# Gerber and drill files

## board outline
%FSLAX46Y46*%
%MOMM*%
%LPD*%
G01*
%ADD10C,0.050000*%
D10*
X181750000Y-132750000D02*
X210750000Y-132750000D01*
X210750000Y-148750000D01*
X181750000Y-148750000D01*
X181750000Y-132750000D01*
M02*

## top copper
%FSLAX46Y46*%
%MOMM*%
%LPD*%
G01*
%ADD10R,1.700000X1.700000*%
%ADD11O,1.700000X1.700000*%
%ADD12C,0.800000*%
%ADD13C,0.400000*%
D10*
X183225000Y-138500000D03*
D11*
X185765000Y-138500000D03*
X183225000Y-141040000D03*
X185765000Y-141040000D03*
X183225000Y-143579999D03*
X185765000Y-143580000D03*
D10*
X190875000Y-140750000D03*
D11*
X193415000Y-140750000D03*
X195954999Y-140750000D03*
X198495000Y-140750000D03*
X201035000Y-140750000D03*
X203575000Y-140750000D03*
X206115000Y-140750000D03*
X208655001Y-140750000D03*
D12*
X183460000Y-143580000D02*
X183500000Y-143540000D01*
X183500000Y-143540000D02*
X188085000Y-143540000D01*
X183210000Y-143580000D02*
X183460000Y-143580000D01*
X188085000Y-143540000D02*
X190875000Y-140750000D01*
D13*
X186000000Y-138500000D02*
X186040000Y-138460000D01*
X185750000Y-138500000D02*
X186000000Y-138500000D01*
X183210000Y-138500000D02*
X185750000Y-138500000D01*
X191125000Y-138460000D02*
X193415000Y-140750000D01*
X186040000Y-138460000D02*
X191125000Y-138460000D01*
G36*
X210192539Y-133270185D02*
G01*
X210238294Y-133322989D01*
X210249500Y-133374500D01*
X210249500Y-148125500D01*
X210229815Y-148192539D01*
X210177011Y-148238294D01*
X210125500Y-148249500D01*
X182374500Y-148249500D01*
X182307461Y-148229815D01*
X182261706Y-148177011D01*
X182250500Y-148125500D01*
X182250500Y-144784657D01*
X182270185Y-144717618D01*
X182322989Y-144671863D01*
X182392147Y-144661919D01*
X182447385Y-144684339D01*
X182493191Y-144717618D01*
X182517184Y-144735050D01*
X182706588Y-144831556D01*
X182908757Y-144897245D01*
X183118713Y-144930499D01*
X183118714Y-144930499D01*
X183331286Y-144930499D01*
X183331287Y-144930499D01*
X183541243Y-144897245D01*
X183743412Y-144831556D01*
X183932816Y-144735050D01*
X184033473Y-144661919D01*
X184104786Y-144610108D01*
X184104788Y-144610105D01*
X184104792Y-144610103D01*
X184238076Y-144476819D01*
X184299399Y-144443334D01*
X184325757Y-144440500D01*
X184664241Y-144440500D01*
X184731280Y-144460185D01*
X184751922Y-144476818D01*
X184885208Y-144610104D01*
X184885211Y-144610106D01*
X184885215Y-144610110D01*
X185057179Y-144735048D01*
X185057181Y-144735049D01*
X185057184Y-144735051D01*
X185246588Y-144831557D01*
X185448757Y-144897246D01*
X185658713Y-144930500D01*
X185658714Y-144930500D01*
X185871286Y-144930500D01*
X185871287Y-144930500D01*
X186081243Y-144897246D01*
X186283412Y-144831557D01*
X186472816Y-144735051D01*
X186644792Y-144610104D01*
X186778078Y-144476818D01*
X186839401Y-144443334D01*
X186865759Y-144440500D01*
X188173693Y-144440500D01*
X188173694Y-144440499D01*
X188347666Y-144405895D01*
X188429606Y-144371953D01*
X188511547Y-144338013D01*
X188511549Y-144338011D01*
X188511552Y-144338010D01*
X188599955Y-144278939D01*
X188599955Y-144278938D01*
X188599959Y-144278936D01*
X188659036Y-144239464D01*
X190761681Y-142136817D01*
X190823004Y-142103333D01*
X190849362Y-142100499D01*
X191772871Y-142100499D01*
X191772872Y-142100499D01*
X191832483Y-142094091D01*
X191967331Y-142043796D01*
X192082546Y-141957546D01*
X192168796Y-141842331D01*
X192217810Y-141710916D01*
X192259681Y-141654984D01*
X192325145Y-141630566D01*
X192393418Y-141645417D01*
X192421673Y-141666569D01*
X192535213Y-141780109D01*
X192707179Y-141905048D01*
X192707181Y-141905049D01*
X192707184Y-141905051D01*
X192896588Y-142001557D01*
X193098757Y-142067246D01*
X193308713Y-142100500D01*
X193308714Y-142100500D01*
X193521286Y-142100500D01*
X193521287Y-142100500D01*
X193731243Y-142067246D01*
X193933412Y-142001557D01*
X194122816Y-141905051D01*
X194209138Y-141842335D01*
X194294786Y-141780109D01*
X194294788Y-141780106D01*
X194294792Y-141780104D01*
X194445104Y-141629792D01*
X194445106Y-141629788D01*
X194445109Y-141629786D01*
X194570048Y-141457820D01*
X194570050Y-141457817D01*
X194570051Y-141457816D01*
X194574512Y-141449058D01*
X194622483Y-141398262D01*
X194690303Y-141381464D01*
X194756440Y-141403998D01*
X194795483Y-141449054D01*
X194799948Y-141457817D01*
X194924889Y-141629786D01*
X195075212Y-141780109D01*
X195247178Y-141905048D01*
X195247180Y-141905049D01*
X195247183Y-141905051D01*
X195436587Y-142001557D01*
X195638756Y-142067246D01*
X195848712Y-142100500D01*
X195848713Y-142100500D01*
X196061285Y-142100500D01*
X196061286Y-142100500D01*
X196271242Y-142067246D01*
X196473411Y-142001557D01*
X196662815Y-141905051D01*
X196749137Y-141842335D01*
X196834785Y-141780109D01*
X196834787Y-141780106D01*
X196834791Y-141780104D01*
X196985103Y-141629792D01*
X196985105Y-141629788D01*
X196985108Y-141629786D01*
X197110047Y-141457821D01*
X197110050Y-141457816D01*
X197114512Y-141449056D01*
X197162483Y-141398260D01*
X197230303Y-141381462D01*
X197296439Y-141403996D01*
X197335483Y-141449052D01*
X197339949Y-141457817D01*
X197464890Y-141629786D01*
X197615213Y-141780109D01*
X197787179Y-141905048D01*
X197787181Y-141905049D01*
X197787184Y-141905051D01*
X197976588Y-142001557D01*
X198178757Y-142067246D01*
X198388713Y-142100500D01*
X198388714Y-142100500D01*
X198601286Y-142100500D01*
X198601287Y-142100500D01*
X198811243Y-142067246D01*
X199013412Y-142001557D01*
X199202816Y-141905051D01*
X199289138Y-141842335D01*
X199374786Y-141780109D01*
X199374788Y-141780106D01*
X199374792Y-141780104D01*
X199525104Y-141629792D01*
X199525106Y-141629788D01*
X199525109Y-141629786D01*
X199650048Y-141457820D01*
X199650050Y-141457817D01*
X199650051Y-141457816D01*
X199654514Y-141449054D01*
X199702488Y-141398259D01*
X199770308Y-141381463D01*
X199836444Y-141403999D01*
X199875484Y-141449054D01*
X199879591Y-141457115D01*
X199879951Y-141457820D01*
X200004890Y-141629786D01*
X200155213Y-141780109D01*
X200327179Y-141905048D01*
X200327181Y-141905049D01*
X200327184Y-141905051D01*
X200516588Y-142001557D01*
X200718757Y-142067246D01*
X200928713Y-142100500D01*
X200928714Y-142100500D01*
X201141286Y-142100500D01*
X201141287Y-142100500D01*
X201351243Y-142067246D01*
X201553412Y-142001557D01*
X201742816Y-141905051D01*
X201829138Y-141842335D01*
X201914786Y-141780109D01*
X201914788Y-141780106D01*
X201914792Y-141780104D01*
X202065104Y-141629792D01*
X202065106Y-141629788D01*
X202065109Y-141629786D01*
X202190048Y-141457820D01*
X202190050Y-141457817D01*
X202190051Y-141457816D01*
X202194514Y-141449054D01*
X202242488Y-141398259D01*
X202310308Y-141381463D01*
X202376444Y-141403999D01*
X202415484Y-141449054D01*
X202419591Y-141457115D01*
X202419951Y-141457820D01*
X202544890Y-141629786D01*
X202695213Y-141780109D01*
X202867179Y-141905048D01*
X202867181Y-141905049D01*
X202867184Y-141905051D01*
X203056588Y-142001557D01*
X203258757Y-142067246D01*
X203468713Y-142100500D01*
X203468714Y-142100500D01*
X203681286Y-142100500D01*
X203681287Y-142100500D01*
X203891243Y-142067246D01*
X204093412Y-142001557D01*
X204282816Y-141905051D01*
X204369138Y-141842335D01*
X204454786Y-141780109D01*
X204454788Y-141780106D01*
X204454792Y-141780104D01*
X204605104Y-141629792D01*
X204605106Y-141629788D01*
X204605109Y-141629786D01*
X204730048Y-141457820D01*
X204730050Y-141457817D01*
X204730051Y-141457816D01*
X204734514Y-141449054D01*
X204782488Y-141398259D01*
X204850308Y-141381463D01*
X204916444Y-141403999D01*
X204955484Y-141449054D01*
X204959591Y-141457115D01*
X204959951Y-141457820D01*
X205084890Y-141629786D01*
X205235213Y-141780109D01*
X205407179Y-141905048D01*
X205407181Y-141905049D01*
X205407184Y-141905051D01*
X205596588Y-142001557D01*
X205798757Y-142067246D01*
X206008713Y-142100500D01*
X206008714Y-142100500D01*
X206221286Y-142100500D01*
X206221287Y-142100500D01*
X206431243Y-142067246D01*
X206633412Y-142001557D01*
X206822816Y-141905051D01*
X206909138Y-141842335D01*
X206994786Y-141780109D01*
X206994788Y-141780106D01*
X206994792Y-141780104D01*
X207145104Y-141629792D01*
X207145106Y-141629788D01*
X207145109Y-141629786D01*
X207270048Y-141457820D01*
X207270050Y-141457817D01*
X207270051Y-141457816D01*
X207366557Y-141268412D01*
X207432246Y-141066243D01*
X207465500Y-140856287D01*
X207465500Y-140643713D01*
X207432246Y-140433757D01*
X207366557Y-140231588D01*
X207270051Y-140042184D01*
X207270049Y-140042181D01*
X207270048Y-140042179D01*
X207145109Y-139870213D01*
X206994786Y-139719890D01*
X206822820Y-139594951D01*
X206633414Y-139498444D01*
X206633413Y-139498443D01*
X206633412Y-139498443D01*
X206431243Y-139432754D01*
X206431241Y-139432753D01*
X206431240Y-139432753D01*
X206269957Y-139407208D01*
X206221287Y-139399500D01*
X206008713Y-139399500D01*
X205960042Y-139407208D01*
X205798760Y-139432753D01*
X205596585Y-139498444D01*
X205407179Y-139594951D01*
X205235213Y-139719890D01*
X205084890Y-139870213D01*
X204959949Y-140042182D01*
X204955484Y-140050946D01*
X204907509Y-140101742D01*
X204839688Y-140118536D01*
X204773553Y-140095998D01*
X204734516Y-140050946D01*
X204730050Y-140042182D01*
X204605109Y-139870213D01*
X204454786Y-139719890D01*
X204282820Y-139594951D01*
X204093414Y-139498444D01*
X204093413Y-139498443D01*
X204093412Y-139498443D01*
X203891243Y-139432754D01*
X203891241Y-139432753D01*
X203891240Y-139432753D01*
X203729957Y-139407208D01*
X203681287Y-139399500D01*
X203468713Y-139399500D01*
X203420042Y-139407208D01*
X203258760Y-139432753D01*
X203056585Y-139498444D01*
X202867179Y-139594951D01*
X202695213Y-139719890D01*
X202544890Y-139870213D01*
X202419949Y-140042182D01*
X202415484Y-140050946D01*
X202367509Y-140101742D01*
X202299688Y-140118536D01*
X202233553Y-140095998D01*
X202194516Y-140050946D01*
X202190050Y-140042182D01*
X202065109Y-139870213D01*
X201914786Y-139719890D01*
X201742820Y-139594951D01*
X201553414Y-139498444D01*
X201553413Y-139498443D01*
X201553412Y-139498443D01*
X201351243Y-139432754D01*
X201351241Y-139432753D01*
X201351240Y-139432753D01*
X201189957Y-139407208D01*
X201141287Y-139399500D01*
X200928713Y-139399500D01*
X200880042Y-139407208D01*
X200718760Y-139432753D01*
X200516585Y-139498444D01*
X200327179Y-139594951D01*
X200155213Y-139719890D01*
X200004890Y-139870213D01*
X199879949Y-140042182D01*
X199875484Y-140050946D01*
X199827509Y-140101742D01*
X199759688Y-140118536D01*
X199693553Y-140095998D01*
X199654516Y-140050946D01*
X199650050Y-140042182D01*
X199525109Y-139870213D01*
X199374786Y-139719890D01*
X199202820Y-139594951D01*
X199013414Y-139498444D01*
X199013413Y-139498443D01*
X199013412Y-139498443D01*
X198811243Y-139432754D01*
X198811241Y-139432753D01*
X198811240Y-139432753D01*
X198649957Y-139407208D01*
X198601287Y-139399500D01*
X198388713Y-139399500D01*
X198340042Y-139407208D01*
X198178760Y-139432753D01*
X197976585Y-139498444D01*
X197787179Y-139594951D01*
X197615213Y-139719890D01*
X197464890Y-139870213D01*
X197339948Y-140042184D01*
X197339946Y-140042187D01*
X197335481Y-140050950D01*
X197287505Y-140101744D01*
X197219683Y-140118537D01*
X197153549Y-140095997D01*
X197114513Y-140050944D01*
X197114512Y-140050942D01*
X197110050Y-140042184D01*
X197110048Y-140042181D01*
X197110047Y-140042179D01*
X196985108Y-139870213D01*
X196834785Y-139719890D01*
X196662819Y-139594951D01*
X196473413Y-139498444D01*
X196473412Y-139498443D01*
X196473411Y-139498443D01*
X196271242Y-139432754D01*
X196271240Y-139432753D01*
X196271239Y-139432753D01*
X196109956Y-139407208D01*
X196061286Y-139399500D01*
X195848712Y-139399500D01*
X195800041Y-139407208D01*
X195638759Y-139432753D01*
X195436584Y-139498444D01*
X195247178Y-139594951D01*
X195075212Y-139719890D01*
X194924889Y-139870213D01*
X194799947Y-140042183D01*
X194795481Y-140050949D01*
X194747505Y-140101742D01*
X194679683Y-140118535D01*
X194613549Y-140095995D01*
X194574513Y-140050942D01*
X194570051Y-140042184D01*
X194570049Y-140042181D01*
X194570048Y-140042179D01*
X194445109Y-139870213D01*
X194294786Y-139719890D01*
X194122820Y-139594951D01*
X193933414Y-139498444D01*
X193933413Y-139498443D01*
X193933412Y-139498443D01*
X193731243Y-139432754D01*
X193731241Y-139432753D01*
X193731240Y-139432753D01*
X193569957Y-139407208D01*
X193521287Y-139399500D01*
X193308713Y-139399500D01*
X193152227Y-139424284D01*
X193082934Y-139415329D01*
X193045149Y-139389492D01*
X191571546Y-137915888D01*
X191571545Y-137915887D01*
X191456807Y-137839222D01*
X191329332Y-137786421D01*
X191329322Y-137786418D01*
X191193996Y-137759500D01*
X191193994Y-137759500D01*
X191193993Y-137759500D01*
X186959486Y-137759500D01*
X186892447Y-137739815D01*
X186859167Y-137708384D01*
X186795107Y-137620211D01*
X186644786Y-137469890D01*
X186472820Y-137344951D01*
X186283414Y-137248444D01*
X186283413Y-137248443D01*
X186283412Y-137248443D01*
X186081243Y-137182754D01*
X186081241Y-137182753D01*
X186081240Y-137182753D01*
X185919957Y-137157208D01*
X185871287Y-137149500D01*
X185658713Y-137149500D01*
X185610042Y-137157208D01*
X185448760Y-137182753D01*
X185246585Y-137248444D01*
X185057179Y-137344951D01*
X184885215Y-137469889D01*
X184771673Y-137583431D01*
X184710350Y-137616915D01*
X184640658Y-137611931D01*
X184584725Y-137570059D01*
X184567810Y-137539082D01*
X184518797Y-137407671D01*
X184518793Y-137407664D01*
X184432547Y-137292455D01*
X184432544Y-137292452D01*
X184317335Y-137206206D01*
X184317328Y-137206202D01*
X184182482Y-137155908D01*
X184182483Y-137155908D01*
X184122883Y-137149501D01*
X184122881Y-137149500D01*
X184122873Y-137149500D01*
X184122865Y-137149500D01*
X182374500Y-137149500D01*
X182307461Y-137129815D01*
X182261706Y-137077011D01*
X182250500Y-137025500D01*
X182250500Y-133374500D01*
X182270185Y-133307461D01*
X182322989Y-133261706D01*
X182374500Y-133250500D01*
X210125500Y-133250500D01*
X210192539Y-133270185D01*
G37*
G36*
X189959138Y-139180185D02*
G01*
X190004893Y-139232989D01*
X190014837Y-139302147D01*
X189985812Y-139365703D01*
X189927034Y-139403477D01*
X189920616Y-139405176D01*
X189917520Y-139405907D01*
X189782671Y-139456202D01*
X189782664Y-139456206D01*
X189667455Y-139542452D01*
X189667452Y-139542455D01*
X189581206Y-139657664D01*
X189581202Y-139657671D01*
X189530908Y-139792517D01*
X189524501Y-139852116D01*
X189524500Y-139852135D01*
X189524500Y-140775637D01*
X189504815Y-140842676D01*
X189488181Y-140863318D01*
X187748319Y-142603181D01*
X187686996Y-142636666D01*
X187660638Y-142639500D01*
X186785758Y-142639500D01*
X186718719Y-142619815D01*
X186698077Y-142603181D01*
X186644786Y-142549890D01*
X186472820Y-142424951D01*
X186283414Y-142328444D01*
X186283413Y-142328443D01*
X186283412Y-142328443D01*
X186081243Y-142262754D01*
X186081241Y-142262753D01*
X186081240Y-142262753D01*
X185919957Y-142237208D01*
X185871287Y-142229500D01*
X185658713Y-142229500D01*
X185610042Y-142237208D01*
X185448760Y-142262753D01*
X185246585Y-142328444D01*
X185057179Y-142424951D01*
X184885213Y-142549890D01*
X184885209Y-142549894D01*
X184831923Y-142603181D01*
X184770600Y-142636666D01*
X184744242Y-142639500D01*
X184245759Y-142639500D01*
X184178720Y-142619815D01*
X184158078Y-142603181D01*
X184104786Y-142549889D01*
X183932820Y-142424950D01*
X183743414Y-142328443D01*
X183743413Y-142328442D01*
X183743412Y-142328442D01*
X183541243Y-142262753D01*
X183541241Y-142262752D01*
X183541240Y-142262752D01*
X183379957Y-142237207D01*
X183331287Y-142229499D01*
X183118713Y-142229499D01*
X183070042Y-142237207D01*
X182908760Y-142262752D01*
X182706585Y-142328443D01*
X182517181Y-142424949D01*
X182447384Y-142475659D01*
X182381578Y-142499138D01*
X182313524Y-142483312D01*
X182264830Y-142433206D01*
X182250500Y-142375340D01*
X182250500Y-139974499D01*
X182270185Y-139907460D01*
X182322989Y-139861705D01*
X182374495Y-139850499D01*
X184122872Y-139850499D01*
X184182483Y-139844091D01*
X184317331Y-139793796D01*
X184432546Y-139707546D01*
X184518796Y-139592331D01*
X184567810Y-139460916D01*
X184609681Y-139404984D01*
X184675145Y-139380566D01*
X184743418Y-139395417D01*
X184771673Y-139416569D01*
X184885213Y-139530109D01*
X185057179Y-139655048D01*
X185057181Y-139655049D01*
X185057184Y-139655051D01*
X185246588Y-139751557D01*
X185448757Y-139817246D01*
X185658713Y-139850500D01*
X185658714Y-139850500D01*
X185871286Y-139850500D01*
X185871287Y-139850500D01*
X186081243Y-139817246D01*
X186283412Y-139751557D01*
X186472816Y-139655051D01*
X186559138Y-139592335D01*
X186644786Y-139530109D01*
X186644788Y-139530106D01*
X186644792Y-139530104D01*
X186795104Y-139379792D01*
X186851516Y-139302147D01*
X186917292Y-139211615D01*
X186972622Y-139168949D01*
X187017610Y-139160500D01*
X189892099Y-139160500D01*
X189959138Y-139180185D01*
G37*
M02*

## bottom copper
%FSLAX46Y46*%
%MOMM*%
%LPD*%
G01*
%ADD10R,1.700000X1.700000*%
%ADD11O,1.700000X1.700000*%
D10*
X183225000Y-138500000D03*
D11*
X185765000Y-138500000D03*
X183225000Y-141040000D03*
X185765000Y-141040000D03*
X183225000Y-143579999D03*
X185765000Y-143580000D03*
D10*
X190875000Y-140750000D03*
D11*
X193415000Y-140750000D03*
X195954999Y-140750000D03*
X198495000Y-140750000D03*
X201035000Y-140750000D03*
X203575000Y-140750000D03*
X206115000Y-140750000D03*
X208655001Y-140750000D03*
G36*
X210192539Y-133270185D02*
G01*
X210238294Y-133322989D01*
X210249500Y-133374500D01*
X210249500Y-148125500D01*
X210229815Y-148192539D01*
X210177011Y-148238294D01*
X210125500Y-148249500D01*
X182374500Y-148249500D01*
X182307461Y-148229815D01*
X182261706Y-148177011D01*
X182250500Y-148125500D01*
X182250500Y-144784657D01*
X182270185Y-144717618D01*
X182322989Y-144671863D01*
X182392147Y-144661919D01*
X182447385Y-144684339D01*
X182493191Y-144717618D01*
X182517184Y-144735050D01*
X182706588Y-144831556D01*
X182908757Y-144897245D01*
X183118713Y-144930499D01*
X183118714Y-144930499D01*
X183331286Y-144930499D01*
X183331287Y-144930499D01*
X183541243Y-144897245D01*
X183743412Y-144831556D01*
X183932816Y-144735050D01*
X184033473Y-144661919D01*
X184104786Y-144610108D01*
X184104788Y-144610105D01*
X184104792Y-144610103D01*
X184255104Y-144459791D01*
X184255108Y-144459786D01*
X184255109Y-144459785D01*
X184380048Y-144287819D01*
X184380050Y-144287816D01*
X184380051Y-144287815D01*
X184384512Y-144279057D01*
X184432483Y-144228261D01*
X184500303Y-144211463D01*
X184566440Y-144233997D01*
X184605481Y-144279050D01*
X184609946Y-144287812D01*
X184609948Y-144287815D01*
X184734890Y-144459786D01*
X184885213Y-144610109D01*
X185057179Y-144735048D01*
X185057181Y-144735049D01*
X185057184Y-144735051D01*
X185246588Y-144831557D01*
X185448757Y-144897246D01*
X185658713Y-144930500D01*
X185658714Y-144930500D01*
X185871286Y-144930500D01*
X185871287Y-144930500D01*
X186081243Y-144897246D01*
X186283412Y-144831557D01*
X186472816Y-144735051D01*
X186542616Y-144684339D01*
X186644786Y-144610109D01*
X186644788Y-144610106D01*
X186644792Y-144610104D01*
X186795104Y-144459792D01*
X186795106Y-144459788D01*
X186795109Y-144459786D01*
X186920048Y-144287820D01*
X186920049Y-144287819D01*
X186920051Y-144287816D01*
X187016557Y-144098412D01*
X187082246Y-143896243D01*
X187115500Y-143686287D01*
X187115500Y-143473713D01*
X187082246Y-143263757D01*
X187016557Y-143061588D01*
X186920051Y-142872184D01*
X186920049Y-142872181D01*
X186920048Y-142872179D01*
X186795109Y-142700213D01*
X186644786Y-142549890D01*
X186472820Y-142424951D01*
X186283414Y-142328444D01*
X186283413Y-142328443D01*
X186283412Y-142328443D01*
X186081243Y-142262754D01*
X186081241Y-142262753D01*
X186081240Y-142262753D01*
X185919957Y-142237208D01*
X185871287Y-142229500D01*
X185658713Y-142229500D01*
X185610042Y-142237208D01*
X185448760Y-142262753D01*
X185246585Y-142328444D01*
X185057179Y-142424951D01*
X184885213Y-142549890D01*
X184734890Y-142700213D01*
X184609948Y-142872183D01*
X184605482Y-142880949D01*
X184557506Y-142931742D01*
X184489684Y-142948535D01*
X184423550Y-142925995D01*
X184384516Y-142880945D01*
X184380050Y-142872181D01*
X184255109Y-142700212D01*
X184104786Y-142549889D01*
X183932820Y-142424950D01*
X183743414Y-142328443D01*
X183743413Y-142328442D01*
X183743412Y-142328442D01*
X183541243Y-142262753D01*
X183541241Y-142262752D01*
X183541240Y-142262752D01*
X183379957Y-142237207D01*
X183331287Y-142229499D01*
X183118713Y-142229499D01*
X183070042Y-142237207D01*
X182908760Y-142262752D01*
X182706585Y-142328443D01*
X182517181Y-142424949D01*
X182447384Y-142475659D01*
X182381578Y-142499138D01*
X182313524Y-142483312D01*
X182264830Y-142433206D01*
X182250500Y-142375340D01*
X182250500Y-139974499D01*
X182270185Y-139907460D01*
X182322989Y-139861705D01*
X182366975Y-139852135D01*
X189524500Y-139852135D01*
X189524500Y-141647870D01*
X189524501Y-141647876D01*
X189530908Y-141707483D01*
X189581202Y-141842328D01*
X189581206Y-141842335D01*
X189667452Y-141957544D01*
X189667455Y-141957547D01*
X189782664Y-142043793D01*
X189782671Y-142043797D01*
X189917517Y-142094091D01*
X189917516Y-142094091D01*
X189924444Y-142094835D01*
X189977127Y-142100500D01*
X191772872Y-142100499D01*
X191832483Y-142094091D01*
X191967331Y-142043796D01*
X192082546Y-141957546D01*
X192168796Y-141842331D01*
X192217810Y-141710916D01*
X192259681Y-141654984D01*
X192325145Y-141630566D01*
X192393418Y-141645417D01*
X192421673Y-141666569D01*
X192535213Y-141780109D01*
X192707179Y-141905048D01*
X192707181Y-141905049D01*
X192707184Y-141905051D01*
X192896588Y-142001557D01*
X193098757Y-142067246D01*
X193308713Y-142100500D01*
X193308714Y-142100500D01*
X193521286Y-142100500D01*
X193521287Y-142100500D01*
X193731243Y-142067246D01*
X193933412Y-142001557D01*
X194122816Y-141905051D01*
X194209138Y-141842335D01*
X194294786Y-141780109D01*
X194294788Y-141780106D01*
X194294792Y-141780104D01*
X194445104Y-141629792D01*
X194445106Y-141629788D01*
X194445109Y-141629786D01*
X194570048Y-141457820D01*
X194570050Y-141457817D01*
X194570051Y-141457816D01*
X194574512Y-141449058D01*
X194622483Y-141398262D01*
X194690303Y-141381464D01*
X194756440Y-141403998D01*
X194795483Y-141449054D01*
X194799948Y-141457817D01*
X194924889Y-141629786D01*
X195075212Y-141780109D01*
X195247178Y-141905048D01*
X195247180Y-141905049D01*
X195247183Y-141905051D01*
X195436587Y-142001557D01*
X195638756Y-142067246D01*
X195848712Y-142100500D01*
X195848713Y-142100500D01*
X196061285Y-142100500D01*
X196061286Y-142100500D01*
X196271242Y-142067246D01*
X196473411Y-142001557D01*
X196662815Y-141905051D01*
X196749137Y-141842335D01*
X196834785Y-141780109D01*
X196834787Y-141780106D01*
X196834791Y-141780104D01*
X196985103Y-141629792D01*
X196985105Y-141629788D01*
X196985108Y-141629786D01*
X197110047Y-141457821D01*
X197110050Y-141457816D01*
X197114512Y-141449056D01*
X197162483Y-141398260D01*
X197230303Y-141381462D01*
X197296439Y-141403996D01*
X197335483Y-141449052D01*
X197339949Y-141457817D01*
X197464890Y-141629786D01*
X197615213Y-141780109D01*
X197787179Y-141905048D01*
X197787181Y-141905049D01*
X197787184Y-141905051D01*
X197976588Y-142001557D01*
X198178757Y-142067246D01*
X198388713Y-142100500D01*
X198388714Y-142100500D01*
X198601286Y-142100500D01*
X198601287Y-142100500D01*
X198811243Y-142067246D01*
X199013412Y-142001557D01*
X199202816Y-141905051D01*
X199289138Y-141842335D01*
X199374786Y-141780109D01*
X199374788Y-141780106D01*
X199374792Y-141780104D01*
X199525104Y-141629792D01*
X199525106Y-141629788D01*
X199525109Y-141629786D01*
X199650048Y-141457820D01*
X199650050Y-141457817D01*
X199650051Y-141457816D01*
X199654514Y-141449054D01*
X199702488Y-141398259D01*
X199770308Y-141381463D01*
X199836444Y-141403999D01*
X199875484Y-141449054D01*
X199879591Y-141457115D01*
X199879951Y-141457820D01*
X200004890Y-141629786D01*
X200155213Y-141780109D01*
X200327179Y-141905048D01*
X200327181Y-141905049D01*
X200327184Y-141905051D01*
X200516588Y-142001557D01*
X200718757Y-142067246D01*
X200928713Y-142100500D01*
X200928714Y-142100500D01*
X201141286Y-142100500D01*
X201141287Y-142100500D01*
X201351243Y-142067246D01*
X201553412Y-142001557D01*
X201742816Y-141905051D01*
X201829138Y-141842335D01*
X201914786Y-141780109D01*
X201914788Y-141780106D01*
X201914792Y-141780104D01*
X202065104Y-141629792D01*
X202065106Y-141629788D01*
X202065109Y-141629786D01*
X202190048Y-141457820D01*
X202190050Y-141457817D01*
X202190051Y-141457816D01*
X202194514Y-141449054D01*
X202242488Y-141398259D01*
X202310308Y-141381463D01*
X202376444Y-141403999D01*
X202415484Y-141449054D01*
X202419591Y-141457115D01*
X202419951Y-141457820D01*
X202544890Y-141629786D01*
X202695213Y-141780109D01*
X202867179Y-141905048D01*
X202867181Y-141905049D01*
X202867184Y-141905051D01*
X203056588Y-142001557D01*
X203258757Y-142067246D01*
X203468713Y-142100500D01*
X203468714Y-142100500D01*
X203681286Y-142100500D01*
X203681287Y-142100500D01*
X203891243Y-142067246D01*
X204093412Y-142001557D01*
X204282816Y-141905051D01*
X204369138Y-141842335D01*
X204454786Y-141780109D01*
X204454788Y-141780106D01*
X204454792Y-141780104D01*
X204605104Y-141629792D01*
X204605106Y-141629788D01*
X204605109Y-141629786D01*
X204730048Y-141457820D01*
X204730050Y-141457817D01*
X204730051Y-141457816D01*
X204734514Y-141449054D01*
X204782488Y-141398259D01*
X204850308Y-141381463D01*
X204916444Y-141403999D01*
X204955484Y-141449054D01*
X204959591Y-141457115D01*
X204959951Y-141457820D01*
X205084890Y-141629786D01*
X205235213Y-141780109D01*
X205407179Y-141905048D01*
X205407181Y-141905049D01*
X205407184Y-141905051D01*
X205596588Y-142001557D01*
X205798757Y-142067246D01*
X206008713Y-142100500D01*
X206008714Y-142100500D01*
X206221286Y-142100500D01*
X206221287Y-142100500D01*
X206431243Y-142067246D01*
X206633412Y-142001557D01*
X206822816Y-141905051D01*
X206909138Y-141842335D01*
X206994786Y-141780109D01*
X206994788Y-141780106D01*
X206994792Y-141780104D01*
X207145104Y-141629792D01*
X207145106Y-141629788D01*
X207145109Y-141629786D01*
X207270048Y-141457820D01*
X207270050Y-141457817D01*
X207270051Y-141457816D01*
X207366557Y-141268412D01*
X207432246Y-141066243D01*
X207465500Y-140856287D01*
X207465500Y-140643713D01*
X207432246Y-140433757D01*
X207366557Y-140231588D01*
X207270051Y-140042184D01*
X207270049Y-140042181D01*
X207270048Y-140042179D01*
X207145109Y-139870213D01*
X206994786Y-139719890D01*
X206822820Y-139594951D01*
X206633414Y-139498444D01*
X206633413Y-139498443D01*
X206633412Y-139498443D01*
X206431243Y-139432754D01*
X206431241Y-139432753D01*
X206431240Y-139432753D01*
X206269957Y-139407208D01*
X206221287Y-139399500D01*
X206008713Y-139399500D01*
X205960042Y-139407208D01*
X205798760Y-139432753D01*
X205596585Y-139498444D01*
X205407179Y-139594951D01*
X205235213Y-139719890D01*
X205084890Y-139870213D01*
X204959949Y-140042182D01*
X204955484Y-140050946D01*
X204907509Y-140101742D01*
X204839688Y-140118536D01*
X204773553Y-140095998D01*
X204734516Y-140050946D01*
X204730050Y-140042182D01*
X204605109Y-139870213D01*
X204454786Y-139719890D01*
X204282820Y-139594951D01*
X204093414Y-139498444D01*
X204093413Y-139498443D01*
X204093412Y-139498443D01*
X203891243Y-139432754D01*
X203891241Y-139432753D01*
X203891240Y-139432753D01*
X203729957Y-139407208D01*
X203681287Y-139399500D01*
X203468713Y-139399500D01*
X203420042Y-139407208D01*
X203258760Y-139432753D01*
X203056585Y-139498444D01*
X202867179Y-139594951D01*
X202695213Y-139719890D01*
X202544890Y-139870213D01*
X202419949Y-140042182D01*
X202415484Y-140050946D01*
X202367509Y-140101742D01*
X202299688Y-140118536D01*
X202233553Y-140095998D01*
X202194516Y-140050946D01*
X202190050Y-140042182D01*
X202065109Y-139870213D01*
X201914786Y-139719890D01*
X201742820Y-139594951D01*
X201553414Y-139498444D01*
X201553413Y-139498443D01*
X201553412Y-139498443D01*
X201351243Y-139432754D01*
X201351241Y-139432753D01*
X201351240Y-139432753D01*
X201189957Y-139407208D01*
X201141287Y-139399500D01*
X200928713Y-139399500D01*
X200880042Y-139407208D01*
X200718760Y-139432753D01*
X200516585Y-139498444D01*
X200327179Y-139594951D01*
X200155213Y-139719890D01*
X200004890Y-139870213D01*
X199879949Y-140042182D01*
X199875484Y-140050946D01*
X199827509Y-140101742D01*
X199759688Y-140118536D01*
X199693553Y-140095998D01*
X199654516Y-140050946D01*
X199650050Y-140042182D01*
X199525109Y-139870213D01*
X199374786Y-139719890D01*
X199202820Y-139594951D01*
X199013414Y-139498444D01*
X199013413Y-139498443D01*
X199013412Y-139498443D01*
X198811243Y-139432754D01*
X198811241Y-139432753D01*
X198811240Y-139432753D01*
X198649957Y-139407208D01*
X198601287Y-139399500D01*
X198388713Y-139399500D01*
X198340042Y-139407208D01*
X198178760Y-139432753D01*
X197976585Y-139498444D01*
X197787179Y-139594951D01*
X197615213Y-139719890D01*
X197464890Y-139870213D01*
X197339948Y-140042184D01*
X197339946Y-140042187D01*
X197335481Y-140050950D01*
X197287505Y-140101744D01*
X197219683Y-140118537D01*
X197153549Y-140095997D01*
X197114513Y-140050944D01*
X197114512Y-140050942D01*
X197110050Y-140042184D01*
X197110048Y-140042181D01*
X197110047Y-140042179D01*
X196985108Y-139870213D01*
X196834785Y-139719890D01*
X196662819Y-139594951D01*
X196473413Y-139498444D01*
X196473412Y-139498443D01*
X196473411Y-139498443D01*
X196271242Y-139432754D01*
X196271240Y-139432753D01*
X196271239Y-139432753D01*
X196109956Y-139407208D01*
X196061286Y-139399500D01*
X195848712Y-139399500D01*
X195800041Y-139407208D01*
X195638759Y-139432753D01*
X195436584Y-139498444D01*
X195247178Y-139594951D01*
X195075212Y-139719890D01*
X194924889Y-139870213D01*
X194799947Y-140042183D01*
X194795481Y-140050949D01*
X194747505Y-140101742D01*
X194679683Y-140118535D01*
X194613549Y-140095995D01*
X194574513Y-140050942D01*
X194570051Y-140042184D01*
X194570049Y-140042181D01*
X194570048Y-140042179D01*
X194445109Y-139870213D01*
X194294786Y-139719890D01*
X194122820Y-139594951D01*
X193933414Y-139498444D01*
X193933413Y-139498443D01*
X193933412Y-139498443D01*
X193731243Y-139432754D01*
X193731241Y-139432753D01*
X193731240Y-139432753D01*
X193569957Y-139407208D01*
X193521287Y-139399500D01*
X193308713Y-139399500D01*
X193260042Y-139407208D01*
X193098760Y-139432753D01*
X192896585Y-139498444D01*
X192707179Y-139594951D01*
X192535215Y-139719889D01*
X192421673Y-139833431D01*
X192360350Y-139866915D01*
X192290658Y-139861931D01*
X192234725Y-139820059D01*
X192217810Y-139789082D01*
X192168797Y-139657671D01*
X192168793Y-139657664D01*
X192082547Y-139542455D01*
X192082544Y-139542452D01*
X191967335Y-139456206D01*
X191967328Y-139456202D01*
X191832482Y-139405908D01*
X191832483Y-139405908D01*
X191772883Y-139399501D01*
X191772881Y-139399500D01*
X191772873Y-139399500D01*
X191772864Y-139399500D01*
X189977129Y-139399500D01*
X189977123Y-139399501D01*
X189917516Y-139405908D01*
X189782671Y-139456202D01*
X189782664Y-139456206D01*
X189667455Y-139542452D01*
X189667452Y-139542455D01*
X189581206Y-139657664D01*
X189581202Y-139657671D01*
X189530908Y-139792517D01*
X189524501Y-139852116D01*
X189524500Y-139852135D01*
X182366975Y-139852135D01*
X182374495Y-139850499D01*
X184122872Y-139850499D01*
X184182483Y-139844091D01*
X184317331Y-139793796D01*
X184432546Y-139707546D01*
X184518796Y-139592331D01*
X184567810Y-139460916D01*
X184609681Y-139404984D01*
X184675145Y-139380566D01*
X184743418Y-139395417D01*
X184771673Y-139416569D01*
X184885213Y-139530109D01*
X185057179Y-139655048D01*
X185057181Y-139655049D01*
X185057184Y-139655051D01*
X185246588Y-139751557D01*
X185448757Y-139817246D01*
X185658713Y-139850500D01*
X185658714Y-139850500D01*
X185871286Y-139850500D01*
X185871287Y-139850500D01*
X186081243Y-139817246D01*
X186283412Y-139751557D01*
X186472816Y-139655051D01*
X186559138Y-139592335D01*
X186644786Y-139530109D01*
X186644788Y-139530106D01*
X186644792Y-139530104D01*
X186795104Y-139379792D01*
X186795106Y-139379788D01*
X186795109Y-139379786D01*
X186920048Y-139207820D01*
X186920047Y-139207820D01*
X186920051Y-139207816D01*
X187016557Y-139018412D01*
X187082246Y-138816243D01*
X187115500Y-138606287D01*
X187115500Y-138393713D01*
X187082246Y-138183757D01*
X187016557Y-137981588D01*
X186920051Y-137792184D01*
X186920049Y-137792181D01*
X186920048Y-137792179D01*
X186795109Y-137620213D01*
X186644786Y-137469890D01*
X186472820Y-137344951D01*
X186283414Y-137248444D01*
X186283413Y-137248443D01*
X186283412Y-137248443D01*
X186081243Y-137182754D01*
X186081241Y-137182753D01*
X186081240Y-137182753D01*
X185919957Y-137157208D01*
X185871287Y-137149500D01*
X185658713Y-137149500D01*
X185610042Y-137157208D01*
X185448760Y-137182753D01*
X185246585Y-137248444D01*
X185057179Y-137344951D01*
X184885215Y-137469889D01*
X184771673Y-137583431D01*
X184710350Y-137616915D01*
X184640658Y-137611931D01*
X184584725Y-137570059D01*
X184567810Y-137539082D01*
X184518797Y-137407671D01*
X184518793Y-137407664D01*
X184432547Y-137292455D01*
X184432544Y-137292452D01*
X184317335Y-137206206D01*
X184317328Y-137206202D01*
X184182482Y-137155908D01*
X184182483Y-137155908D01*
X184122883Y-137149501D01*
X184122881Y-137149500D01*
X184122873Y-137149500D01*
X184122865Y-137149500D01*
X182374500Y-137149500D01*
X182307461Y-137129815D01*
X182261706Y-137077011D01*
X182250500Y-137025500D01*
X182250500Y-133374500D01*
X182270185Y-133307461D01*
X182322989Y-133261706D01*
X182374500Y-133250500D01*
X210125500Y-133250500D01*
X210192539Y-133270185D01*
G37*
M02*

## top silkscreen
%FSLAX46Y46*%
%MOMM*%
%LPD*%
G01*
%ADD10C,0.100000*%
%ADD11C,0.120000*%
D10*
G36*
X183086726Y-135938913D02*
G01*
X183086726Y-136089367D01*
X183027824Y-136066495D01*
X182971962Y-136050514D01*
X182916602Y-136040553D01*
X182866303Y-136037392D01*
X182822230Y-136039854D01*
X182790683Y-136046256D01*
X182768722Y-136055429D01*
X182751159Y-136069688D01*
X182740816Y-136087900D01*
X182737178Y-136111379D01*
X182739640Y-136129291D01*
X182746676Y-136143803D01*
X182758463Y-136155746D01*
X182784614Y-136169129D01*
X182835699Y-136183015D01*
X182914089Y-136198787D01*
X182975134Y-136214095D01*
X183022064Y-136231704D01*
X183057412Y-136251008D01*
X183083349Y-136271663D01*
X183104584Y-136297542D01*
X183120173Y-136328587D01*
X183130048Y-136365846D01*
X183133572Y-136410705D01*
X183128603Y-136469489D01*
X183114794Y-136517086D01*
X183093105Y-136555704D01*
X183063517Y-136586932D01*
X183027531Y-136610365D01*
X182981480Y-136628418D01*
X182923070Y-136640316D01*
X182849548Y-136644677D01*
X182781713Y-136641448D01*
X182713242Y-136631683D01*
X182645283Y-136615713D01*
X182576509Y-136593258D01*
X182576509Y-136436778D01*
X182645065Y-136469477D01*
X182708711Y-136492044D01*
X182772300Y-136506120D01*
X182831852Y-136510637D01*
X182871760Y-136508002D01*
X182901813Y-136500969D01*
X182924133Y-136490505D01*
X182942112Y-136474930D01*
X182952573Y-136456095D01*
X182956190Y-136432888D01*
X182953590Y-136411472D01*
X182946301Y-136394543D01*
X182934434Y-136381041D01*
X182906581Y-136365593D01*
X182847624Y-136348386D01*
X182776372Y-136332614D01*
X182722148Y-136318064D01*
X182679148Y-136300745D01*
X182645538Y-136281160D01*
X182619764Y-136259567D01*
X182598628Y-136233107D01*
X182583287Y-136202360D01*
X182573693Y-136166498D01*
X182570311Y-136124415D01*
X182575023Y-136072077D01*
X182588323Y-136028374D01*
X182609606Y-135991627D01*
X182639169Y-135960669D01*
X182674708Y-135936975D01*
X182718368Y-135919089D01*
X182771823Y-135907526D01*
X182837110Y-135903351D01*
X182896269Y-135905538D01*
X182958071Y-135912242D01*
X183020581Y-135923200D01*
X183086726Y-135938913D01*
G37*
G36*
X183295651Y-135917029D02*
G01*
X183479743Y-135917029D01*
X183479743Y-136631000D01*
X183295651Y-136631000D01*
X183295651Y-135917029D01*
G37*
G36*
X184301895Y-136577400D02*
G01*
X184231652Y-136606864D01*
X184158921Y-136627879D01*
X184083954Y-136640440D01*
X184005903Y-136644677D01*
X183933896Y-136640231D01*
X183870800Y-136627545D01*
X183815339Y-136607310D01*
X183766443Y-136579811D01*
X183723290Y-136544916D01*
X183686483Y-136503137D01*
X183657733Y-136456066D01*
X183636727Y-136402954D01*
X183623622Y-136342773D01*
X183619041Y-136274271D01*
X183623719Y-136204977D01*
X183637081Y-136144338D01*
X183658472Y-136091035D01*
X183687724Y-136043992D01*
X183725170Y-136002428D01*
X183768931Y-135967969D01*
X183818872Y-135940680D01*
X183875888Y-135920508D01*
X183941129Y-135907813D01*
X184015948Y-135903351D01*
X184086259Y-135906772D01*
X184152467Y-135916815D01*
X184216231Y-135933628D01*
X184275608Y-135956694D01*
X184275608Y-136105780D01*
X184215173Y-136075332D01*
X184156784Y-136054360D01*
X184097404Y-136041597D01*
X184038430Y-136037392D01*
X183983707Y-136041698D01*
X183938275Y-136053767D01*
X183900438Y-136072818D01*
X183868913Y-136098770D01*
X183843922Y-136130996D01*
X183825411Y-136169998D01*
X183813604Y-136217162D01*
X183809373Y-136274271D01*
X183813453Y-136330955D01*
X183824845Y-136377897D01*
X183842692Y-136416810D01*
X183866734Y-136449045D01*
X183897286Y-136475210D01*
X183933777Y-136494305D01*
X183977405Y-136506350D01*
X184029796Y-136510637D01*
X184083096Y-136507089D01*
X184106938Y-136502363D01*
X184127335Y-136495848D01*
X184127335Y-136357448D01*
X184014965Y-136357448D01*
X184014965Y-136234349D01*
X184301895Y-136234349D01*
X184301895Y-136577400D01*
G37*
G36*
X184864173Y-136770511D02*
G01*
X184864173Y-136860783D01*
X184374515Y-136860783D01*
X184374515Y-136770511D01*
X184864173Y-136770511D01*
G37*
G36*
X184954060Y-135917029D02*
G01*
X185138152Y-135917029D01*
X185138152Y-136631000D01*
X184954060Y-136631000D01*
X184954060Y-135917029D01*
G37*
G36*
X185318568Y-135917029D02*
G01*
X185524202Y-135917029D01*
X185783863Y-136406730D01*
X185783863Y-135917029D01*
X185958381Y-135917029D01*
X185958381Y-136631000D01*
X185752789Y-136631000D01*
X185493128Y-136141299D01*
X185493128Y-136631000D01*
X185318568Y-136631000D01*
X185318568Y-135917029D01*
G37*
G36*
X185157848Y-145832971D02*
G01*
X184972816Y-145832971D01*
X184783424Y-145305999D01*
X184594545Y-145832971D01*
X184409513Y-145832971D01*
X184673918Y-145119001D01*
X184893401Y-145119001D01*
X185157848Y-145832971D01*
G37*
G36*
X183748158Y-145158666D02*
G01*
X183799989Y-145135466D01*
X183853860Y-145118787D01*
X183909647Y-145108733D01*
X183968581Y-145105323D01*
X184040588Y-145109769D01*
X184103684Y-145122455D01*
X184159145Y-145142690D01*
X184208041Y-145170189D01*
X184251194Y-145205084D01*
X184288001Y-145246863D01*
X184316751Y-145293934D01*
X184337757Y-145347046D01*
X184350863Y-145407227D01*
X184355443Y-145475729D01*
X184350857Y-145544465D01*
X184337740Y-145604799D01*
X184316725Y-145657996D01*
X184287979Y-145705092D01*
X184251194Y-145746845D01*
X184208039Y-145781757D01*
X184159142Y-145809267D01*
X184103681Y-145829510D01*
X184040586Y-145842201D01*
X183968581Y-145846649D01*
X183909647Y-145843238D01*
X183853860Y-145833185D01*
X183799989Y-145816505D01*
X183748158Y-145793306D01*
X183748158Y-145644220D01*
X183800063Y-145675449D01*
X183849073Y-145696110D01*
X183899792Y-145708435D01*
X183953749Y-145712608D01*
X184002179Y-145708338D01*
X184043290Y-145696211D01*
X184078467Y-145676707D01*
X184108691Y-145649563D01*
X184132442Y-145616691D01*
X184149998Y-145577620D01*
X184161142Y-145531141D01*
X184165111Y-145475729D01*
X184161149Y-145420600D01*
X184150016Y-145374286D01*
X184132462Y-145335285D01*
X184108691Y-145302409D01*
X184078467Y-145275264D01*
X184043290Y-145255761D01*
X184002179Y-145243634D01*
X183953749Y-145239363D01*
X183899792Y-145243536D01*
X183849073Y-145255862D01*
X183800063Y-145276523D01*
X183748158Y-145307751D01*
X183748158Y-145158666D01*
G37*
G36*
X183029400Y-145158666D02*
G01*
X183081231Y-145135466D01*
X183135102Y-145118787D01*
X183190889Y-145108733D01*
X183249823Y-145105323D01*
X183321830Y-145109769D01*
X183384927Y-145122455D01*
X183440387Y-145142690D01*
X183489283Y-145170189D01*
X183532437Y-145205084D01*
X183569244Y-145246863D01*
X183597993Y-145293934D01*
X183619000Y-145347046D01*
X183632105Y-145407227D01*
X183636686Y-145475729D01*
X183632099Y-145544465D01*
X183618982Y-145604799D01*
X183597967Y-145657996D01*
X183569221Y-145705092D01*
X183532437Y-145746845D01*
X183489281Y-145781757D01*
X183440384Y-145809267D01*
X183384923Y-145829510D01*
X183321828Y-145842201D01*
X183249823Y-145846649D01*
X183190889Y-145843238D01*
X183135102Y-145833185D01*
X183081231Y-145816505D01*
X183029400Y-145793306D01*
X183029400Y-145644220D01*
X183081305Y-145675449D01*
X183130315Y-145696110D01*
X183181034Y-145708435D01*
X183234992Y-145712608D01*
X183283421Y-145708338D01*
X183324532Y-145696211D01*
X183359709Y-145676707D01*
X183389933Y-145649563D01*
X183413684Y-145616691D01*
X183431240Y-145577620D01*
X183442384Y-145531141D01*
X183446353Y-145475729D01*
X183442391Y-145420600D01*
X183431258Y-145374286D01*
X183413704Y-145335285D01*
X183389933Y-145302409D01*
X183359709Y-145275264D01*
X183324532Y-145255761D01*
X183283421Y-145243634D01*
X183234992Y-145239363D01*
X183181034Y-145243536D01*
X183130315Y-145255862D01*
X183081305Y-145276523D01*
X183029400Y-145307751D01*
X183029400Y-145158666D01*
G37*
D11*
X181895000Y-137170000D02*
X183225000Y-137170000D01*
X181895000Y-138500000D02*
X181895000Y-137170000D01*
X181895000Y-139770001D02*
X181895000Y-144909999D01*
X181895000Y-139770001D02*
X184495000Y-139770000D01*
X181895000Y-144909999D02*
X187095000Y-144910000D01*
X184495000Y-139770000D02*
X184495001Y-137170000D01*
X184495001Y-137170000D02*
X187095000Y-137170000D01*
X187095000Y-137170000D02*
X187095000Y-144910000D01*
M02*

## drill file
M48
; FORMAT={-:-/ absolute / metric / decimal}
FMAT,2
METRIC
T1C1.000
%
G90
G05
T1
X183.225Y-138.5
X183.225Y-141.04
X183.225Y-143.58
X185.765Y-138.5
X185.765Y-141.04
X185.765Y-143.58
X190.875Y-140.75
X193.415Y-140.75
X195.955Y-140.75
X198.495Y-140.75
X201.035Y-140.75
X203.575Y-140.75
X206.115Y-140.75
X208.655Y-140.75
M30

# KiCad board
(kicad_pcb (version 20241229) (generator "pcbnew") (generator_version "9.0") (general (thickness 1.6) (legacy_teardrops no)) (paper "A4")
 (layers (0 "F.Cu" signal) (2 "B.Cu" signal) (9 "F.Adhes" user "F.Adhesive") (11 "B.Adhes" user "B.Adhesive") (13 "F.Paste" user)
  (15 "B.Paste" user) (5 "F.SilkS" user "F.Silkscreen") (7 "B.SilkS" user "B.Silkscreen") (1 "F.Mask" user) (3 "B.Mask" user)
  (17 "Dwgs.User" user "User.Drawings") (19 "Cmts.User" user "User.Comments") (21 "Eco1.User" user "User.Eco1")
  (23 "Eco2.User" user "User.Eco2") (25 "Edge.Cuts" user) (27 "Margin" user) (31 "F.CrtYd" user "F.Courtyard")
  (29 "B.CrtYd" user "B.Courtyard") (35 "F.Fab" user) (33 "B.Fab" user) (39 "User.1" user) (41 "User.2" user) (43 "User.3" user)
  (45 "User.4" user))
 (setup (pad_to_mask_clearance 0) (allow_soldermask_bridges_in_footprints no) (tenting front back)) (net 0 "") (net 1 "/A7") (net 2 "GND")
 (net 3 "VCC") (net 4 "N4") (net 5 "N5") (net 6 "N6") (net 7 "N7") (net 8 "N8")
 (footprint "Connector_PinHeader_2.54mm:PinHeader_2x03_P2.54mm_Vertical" (layer "F.Cu") (at 183.225 138.5)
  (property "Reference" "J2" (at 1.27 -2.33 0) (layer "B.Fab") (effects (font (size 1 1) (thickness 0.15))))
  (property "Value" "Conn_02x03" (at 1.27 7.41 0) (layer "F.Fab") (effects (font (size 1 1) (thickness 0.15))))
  (fp_line (start -1.33 -1.33) (end 0 -1.33) (stroke (width 0.12) (type solid)) (layer "F.SilkS"))
  (fp_line (start -1.33 0) (end -1.33 -1.33) (stroke (width 0.12) (type solid)) (layer "F.SilkS"))
  (fp_line (start -1.33 1.270001) (end -1.33 6.409999) (stroke (width 0.12) (type solid)) (layer "F.SilkS"))
  (fp_line (start -1.33 1.270001) (end 1.27 1.27) (stroke (width 0.12) (type solid)) (layer "F.SilkS"))
  (fp_line (start -1.33 6.409999) (end 3.87 6.41) (stroke (width 0.12) (type solid)) (layer "F.SilkS"))
  (fp_line (start 1.27 1.27) (end 1.270001 -1.33) (stroke (width 0.12) (type solid)) (layer "F.SilkS"))
  (fp_line (start 1.270001 -1.33) (end 3.87 -1.33) (stroke (width 0.12) (type solid)) (layer "F.SilkS"))
  (fp_line (start 3.87 -1.33) (end 3.87 6.41) (stroke (width 0.12) (type solid)) (layer "F.SilkS"))
  (pad "1" thru_hole rect (at 0 0) (size 1.7 1.7) (drill 1) (layers "*.Cu" "*.Mask") (remove_unused_layers no) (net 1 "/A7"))
  (pad "2" thru_hole oval (at 2.54 0) (size 1.7 1.7) (drill 1) (layers "*.Cu" "*.Mask") (remove_unused_layers no) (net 1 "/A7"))
  (pad "3" thru_hole oval (at 0 2.54) (size 1.7 1.7) (drill 1) (layers "*.Cu" "*.Mask") (remove_unused_layers no) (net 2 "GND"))
  (pad "4" thru_hole oval (at 2.54 2.54) (size 1.7 1.7) (drill 1) (layers "*.Cu" "*.Mask") (remove_unused_layers no) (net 2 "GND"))
  (pad "5" thru_hole oval (at 0 5.079999) (size 1.7 1.7) (drill 1) (layers "*.Cu" "*.Mask") (remove_unused_layers no) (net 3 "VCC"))
  (pad "6" thru_hole oval (at 2.54 5.08) (size 1.7 1.7) (drill 1) (layers "*.Cu" "*.Mask") (remove_unused_layers no) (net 3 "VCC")))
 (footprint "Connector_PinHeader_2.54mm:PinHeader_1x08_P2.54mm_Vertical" (layer "B.Cu") (at 190.875 140.75 -90)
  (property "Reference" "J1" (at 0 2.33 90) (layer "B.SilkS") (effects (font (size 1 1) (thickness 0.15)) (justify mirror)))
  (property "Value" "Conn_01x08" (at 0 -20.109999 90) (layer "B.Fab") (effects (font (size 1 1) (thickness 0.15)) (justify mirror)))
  (pad "1" thru_hole rect (at 0 0 270) (size 1.7 1.7) (drill 1) (layers "*.Cu" "*.Mask") (remove_unused_layers no) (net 3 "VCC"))
  (pad "2" thru_hole oval (at 0 -2.54 270) (size 1.7 1.7) (drill 1) (layers "*.Cu" "*.Mask") (remove_unused_layers no) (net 1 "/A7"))
  (pad "3" thru_hole oval (at 0 -5.079999 270) (size 1.7 1.7) (drill 1) (layers "*.Cu" "*.Mask") (remove_unused_layers no) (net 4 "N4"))
  (pad "4" thru_hole oval (at 0 -7.62 270) (size 1.7 1.7) (drill 1) (layers "*.Cu" "*.Mask") (remove_unused_layers no) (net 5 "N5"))
  (pad "5" thru_hole oval (at 0 -10.16 270) (size 1.7 1.7) (drill 1) (layers "*.Cu" "*.Mask") (remove_unused_layers no) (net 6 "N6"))
  (pad "6" thru_hole oval (at 0 -12.7 270) (size 1.7 1.7) (drill 1) (layers "*.Cu" "*.Mask") (remove_unused_layers no) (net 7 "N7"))
  (pad "7" thru_hole oval (at 0 -15.24 270) (size 1.7 1.7) (drill 1) (layers "*.Cu" "*.Mask") (remove_unused_layers no) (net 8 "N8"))
  (pad "8" thru_hole oval (at 0 -17.780001 270) (size 1.7 1.7) (drill 1) (layers "*.Cu" "*.Mask") (remove_unused_layers no) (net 2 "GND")))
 (gr_rect (start 181.75 132.75) (end 210.75 148.75) (stroke (width 0.05) (type default)) (fill no) (layer "Edge.Cuts"))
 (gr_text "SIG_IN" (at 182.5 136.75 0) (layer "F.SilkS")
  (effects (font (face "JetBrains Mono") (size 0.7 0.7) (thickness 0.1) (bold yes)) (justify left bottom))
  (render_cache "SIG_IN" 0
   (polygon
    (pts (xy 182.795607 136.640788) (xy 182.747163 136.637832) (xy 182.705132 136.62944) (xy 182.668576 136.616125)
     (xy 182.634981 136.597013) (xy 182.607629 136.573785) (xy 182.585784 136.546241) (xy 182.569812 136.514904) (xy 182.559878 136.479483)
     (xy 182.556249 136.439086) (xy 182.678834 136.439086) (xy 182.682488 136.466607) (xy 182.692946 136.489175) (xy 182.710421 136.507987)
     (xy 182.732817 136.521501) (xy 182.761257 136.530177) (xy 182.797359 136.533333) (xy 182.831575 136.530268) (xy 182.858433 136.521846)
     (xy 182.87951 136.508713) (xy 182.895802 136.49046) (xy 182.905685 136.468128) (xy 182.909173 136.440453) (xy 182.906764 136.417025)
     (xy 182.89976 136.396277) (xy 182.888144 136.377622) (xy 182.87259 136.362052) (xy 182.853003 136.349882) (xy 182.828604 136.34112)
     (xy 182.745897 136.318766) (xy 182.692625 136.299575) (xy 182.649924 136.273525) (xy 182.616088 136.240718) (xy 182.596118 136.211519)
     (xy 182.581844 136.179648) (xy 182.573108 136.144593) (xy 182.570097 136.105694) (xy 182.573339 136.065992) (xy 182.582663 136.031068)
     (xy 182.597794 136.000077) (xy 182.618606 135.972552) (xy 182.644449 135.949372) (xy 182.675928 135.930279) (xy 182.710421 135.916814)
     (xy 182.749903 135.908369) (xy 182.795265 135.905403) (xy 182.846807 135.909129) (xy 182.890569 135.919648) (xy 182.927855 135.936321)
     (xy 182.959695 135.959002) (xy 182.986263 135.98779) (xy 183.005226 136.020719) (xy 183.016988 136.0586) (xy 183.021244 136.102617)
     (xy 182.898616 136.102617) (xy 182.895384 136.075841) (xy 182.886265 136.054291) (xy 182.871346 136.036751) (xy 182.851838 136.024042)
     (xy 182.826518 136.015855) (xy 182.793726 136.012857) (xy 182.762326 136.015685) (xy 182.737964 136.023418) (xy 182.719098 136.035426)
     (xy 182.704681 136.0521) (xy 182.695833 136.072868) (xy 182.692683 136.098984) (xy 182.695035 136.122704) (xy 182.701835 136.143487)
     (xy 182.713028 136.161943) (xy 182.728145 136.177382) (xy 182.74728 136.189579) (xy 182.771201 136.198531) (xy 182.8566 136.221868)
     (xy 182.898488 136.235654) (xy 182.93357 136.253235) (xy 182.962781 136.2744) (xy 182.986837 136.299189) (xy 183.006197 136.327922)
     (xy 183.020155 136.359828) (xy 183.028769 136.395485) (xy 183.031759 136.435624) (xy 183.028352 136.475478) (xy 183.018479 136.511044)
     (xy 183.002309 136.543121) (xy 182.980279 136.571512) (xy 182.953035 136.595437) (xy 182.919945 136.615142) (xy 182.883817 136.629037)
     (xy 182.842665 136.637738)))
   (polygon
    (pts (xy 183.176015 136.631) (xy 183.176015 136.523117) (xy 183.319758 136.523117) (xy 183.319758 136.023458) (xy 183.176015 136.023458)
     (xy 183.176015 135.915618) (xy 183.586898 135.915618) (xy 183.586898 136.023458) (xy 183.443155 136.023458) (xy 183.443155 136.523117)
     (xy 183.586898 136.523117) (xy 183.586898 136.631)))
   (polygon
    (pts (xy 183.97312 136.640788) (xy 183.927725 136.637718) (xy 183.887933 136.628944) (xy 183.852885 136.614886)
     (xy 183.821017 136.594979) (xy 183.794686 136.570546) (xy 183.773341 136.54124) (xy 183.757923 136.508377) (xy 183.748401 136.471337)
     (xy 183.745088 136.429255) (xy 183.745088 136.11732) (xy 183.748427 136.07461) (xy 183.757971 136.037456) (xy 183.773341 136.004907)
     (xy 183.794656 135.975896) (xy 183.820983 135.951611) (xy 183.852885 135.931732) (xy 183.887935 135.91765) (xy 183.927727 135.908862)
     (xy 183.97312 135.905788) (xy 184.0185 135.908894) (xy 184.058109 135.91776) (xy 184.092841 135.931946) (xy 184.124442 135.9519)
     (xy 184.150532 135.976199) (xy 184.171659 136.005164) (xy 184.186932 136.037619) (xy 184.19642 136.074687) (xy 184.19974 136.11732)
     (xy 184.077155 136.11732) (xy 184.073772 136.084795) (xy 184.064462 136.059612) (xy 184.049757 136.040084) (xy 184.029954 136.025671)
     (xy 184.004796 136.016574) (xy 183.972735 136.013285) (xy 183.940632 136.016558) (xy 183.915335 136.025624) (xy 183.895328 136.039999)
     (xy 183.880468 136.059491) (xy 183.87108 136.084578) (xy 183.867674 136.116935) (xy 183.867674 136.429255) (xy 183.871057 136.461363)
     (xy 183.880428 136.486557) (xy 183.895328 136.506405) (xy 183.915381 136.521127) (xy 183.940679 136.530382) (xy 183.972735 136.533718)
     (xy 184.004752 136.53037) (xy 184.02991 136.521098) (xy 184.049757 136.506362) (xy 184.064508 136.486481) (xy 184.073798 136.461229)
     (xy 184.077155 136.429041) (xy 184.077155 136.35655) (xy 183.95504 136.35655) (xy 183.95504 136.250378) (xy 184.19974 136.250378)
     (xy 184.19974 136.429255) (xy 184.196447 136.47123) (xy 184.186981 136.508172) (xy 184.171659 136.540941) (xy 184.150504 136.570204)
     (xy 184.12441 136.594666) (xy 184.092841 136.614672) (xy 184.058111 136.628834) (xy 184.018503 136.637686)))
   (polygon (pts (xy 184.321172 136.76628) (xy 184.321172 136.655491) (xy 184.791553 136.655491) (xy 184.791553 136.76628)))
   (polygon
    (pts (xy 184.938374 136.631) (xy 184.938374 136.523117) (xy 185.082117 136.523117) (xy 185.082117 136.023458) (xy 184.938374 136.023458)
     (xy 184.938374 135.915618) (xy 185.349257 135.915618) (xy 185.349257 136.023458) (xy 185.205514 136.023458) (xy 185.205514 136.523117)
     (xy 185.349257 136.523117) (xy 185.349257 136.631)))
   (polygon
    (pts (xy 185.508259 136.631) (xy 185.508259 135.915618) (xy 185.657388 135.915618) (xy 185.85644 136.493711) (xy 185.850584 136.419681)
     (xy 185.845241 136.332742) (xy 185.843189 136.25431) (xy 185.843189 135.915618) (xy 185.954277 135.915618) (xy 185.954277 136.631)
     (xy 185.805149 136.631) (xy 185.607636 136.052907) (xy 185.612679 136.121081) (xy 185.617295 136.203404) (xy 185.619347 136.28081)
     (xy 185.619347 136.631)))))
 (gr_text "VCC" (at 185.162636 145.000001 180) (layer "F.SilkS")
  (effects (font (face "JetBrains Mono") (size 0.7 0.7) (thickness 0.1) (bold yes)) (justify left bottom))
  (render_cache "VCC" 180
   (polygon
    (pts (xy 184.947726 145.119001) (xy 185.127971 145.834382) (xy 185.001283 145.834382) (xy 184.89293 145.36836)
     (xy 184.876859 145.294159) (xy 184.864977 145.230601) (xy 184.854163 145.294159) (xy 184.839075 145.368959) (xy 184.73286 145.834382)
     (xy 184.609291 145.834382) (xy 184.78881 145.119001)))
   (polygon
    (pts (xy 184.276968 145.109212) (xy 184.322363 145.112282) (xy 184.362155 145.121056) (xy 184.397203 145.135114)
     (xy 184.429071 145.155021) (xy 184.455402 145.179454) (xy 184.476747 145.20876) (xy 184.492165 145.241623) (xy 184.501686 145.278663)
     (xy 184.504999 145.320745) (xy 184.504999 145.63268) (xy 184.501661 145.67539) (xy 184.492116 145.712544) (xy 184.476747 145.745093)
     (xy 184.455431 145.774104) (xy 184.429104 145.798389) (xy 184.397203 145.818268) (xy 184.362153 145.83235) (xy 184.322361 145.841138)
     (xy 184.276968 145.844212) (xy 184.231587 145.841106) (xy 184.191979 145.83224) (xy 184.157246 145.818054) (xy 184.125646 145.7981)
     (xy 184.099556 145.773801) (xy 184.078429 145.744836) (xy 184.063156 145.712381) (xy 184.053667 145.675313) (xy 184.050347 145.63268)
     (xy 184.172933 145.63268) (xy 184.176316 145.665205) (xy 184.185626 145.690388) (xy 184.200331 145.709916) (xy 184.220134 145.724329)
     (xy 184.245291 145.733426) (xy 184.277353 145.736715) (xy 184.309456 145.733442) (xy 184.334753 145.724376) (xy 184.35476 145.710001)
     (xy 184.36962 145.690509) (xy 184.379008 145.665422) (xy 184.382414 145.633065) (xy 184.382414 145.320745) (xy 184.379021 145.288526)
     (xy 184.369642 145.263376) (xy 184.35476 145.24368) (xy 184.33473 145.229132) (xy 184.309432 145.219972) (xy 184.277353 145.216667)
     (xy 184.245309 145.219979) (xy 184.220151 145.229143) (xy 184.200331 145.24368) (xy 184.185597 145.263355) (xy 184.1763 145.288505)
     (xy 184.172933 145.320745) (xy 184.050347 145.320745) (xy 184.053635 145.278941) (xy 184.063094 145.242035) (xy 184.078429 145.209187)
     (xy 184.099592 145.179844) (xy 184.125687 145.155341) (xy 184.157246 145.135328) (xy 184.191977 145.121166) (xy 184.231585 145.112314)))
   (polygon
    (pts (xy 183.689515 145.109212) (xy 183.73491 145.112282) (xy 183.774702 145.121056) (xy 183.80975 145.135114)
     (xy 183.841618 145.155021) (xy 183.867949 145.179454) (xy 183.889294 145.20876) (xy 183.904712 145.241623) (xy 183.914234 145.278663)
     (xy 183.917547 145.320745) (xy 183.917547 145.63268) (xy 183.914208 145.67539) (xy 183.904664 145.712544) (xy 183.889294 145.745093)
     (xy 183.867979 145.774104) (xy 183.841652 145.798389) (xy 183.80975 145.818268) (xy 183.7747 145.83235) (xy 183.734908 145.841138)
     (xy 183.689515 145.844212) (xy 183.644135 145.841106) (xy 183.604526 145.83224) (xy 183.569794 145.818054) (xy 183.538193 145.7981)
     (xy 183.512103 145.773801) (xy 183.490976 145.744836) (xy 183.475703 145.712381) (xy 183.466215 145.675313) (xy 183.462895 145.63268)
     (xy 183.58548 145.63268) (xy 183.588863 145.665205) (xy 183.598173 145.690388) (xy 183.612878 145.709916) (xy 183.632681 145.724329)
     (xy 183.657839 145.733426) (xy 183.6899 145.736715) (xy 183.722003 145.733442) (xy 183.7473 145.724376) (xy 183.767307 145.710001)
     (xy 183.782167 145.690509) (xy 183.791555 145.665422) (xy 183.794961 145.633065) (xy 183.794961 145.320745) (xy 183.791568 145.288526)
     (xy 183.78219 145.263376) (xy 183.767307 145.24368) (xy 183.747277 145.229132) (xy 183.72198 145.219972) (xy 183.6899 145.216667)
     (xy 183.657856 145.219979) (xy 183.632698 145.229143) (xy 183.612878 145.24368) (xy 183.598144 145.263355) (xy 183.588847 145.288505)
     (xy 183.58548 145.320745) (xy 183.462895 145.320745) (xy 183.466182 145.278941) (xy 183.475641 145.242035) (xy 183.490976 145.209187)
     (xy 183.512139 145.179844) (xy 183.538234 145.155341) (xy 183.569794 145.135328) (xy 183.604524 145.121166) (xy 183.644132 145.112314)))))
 (segment (start 183.46 143.58) (end 183.5 143.54) (width 0.8) (layer "F.Cu") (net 3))
 (segment (start 183.5 143.54) (end 188.085 143.54) (width 0.8) (layer "F.Cu") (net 3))
 (segment (start 183.21 143.58) (end 183.46 143.58) (width 0.8) (layer "F.Cu") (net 3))
 (segment (start 188.085 143.54) (end 190.875 140.75) (width 0.8) (layer "F.Cu") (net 3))
 (segment (start 186 138.5) (end 186.04 138.46) (width 0.4) (layer "F.Cu") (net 1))
 (segment (start 185.75 138.5) (end 186 138.5) (width 0.4) (layer "F.Cu") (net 1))
 (segment (start 183.21 138.5) (end 185.75 138.5) (width 0.4) (layer "F.Cu") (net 1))
 (segment (start 191.125 138.46) (end 193.415 140.75) (width 0.4) (layer "F.Cu") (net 1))
 (segment (start 186.04 138.46) (end 191.125 138.46) (width 0.4) (layer "F.Cu") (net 1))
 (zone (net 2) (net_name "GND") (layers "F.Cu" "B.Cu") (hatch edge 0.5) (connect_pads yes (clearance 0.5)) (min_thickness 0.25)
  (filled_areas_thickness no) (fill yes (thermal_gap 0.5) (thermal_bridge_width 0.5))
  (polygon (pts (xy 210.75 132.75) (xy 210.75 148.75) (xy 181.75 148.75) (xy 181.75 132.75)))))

